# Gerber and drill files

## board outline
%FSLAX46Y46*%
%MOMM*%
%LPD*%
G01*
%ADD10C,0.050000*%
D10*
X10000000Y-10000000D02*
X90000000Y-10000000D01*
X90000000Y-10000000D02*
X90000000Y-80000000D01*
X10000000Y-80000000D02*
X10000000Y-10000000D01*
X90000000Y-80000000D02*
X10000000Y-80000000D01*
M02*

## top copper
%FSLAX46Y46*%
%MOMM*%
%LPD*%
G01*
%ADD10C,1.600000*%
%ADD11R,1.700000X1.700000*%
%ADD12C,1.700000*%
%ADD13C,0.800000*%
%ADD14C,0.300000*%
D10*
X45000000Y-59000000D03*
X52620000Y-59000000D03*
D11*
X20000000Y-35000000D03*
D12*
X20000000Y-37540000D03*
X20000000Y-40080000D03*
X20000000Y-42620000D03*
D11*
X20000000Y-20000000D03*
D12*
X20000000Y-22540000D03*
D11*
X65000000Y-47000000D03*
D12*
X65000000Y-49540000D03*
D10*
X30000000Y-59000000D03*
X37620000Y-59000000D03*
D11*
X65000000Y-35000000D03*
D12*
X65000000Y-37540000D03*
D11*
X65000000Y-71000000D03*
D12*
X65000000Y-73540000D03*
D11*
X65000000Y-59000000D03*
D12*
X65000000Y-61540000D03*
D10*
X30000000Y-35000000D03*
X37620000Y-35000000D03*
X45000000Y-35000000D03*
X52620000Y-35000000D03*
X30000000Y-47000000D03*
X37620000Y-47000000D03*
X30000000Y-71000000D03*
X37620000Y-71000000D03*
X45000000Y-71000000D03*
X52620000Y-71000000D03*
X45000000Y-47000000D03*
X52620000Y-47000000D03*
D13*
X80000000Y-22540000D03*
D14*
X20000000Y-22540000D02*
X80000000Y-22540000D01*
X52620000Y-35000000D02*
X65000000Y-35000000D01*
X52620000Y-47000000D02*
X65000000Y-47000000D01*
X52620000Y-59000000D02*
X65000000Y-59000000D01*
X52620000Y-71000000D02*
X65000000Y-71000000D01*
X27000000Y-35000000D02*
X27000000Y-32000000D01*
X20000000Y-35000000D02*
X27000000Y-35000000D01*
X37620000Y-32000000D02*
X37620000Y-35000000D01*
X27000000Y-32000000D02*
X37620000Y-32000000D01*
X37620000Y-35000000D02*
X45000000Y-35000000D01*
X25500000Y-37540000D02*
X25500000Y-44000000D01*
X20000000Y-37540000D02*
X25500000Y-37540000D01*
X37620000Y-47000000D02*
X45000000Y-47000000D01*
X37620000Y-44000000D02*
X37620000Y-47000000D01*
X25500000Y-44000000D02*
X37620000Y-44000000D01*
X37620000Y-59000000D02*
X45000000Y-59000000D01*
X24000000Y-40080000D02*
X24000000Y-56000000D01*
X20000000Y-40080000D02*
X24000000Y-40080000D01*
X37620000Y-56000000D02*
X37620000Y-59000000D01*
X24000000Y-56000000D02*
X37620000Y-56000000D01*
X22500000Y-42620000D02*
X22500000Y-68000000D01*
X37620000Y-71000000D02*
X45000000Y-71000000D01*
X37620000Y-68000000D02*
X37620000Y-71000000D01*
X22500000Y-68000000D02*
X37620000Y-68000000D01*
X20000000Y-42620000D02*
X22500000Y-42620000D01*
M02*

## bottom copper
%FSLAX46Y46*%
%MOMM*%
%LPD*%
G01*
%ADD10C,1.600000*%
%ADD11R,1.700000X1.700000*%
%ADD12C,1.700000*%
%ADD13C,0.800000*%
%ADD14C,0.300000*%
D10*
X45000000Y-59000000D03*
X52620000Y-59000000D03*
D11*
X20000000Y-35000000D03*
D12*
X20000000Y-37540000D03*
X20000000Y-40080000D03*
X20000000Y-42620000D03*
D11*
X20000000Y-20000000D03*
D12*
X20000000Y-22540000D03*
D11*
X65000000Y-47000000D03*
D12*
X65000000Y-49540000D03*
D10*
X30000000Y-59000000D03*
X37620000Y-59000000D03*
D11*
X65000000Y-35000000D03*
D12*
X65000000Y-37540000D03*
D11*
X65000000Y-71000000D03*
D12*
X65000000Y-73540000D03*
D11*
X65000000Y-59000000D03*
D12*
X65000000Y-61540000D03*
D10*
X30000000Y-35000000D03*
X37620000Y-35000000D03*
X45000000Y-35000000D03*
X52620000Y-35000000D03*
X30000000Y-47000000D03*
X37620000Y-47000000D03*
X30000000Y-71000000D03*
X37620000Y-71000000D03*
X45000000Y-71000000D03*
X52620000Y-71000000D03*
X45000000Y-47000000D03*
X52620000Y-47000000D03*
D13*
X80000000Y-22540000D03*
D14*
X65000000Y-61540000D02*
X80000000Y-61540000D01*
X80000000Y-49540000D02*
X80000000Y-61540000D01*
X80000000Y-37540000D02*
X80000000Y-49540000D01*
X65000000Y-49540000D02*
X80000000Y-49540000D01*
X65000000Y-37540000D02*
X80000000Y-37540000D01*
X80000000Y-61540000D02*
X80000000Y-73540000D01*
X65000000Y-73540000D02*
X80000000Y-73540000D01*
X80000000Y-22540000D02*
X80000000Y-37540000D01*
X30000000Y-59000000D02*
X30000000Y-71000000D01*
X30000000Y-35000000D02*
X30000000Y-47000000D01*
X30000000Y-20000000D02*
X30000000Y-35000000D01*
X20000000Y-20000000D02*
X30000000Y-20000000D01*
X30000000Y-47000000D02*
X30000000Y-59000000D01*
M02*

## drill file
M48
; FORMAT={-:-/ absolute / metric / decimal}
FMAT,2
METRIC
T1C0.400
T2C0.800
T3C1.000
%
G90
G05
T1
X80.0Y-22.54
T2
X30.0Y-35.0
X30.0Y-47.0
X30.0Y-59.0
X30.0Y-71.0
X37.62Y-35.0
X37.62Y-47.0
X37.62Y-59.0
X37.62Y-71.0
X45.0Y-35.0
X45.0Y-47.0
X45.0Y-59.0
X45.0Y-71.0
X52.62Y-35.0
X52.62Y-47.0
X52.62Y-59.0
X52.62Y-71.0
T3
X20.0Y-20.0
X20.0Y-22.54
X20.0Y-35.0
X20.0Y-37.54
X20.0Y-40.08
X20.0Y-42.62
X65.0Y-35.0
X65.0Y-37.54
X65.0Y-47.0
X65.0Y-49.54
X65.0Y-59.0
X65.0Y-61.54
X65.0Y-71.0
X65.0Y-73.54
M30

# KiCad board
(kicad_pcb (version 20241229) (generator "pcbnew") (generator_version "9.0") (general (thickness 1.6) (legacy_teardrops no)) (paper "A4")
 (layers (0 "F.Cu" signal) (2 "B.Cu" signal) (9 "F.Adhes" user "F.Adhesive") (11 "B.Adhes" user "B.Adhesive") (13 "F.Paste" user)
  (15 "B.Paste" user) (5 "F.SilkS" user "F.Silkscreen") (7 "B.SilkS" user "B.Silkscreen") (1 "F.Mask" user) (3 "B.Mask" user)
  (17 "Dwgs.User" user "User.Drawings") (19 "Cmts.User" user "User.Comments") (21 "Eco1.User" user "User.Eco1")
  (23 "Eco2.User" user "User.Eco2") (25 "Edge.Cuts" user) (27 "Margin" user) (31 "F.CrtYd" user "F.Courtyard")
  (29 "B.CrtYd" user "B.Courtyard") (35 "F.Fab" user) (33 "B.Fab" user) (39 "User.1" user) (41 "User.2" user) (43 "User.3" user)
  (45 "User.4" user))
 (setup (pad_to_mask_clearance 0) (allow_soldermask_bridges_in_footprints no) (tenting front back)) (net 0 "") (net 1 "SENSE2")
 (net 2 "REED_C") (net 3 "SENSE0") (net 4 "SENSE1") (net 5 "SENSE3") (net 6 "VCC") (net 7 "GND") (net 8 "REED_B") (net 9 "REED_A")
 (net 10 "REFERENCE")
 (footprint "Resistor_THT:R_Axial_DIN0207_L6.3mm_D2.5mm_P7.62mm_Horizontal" (layer "F.Cu") (at 45 59)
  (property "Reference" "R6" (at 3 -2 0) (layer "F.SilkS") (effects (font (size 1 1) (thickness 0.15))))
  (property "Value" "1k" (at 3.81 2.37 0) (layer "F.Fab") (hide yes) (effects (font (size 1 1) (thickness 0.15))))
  (pad "1" thru_hole circle (at 0 0) (size 1.6 1.6) (drill 0.8) (layers "*.Cu" "*.Mask") (remove_unused_layers no) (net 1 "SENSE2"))
  (pad "2" thru_hole circle (at 7.62 0) (size 1.6 1.6) (drill 0.8) (layers "*.Cu" "*.Mask") (remove_unused_layers no) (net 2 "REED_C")))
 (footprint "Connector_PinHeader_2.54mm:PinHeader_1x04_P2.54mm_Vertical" (layer "F.Cu") (at 20 35)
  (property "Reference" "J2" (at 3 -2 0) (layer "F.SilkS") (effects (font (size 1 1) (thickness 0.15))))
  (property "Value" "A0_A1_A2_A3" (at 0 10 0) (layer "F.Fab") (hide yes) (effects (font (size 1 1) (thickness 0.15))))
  (pad "1" thru_hole rect (at 0 0) (size 1.7 1.7) (drill 1) (layers "*.Cu" "*.Mask") (remove_unused_layers no) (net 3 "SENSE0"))
  (pad "2" thru_hole circle (at 0 2.54) (size 1.7 1.7) (drill 1) (layers "*.Cu" "*.Mask") (remove_unused_layers no) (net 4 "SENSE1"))
  (pad "3" thru_hole circle (at 0 5.08) (size 1.7 1.7) (drill 1) (layers "*.Cu" "*.Mask") (remove_unused_layers no) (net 1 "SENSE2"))
  (pad "4" thru_hole circle (at 0 7.62) (size 1.7 1.7) (drill 1) (layers "*.Cu" "*.Mask") (remove_unused_layers no) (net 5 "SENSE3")))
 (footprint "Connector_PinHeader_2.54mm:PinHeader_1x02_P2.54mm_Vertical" (layer "F.Cu") (at 20 20)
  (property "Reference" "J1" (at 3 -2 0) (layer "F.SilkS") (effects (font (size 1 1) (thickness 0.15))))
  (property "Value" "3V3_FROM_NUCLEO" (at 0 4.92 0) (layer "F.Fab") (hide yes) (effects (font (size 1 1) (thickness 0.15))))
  (pad "1" thru_hole rect (at 0 0) (size 1.7 1.7) (drill 1) (layers "*.Cu" "*.Mask") (remove_unused_layers no) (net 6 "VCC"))
  (pad "2" thru_hole circle (at 0 2.54) (size 1.7 1.7) (drill 1) (layers "*.Cu" "*.Mask") (remove_unused_layers no) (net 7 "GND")))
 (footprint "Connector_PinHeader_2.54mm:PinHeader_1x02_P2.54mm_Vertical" (layer "F.Cu") (at 65 47)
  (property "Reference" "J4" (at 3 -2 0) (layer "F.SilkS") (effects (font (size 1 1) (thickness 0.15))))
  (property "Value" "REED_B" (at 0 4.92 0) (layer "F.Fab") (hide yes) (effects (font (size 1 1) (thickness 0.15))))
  (pad "1" thru_hole rect (at 0 0) (size 1.7 1.7) (drill 1) (layers "*.Cu" "*.Mask") (remove_unused_layers no) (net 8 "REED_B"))
  (pad "2" thru_hole circle (at 0 2.54) (size 1.7 1.7) (drill 1) (layers "*.Cu" "*.Mask") (remove_unused_layers no) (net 7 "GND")))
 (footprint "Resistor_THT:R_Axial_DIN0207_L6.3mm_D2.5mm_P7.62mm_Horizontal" (layer "F.Cu") (at 30 59)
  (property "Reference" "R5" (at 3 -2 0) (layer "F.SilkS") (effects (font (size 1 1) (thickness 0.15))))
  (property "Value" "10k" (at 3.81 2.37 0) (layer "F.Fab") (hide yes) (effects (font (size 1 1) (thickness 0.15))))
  (pad "1" thru_hole circle (at 0 0) (size 1.6 1.6) (drill 0.8) (layers "*.Cu" "*.Mask") (remove_unused_layers no) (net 6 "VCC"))
  (pad "2" thru_hole circle (at 7.62 0) (size 1.6 1.6) (drill 0.8) (layers "*.Cu" "*.Mask") (remove_unused_layers no) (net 1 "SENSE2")))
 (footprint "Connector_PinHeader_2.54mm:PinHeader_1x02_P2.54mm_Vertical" (layer "F.Cu") (at 65 35)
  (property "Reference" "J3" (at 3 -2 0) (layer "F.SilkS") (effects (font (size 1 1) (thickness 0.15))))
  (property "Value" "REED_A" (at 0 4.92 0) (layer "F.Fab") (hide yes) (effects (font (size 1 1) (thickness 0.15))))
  (pad "1" thru_hole rect (at 0 0) (size 1.7 1.7) (drill 1) (layers "*.Cu" "*.Mask") (remove_unused_layers no) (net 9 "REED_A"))
  (pad "2" thru_hole circle (at 0 2.54) (size 1.7 1.7) (drill 1) (layers "*.Cu" "*.Mask") (remove_unused_layers no) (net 7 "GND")))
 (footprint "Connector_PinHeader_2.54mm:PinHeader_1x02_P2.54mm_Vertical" (layer "F.Cu") (at 65 71)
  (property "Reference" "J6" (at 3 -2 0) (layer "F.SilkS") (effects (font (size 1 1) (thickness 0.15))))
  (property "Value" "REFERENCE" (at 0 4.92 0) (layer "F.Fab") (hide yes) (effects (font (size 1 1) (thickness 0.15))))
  (pad "1" thru_hole rect (at 0 0) (size 1.7 1.7) (drill 1) (layers "*.Cu" "*.Mask") (remove_unused_layers no) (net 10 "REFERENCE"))
  (pad "2" thru_hole circle (at 0 2.54) (size 1.7 1.7) (drill 1) (layers "*.Cu" "*.Mask") (remove_unused_layers no) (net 7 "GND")))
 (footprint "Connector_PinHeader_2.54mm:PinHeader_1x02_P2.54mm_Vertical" (layer "F.Cu") (at 65 59)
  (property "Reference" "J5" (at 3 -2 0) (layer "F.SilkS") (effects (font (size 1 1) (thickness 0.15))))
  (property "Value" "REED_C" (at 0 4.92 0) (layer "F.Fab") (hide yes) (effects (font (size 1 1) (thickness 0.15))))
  (pad "1" thru_hole rect (at 0 0) (size 1.7 1.7) (drill 1) (layers "*.Cu" "*.Mask") (remove_unused_layers no) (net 2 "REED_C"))
  (pad "2" thru_hole circle (at 0 2.54) (size 1.7 1.7) (drill 1) (layers "*.Cu" "*.Mask") (remove_unused_layers no) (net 7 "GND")))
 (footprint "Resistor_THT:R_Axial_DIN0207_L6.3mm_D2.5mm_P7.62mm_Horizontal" (layer "F.Cu") (at 30 35)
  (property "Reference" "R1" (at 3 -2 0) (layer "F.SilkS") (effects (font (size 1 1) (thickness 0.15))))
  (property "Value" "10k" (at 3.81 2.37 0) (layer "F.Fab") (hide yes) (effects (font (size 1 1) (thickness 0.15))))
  (pad "1" thru_hole circle (at 0 0) (size 1.6 1.6) (drill 0.8) (layers "*.Cu" "*.Mask") (remove_unused_layers no) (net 6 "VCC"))
  (pad "2" thru_hole circle (at 7.62 0) (size 1.6 1.6) (drill 0.8) (layers "*.Cu" "*.Mask") (remove_unused_layers no) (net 3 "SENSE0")))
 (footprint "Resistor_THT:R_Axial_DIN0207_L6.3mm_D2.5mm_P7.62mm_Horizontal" (layer "F.Cu") (at 45 35)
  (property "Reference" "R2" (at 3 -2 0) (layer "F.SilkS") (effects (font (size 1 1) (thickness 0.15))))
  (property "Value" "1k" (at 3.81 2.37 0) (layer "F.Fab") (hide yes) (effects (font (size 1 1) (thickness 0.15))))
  (pad "1" thru_hole circle (at 0 0) (size 1.6 1.6) (drill 0.8) (layers "*.Cu" "*.Mask") (remove_unused_layers no) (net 3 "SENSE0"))
  (pad "2" thru_hole circle (at 7.62 0) (size 1.6 1.6) (drill 0.8) (layers "*.Cu" "*.Mask") (remove_unused_layers no) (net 9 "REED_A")))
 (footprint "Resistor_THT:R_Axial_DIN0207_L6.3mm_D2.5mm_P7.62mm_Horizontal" (layer "F.Cu") (at 30 47)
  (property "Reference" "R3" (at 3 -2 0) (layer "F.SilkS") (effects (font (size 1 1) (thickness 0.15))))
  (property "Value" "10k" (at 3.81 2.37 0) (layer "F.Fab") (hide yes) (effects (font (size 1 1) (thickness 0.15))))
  (pad "1" thru_hole circle (at 0 0) (size 1.6 1.6) (drill 0.8) (layers "*.Cu" "*.Mask") (remove_unused_layers no) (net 6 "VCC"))
  (pad "2" thru_hole circle (at 7.62 0) (size 1.6 1.6) (drill 0.8) (layers "*.Cu" "*.Mask") (remove_unused_layers no) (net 4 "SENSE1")))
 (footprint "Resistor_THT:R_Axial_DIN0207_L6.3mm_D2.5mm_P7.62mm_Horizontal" (layer "F.Cu") (at 30 71)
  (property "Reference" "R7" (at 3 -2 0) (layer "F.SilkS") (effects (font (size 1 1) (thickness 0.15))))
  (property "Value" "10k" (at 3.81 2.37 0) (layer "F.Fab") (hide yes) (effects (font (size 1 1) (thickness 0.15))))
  (pad "1" thru_hole circle (at 0 0) (size 1.6 1.6) (drill 0.8) (layers "*.Cu" "*.Mask") (remove_unused_layers no) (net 6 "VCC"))
  (pad "2" thru_hole circle (at 7.62 0) (size 1.6 1.6) (drill 0.8) (layers "*.Cu" "*.Mask") (remove_unused_layers no) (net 5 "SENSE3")))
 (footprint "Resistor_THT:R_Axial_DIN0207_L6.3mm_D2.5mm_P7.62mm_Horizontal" (layer "F.Cu") (at 45 71)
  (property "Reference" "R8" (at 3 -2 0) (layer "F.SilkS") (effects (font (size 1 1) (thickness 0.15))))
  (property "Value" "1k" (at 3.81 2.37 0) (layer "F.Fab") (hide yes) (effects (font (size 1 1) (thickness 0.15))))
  (pad "1" thru_hole circle (at 0 0) (size 1.6 1.6) (drill 0.8) (layers "*.Cu" "*.Mask") (remove_unused_layers no) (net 5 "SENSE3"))
  (pad "2" thru_hole circle (at 7.62 0) (size 1.6 1.6) (drill 0.8) (layers "*.Cu" "*.Mask") (remove_unused_layers no) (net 10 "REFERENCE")))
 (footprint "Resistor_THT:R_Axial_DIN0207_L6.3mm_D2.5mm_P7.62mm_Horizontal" (layer "F.Cu") (at 45 47)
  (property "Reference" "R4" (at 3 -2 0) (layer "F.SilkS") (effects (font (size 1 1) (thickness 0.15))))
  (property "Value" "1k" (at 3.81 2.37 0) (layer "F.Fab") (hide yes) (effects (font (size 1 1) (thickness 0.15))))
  (pad "1" thru_hole circle (at 0 0) (size 1.6 1.6) (drill 0.8) (layers "*.Cu" "*.Mask") (remove_unused_layers no) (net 4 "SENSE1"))
  (pad "2" thru_hole circle (at 7.62 0) (size 1.6 1.6) (drill 0.8) (layers "*.Cu" "*.Mask") (remove_unused_layers no) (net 8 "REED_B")))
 (gr_line (start 10 10) (end 90 10) (stroke (width 0.05) (type default)) (layer "Edge.Cuts"))
 (gr_line (start 90 10) (end 90 80) (stroke (width 0.05) (type default)) (layer "Edge.Cuts"))
 (gr_line (start 10 80) (end 10 10) (stroke (width 0.05) (type default)) (layer "Edge.Cuts"))
 (gr_line (start 90 80) (end 10 80) (stroke (width 0.05) (type default)) (layer "Edge.Cuts"))
 (segment (start 20 22.54) (end 80 22.54) (width 0.3) (layer "F.Cu") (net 7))
 (via (at 80 22.54) (size 0.8) (drill 0.4) (layers "F.Cu" "B.Cu") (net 7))
 (segment (start 65 61.54) (end 80 61.54) (width 0.3) (layer "B.Cu") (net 7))
 (segment (start 80 49.54) (end 80 61.54) (width 0.3) (layer "B.Cu") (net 7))
 (segment (start 80 37.54) (end 80 49.54) (width 0.3) (layer "B.Cu") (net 7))
 (segment (start 65 49.54) (end 80 49.54) (width 0.3) (layer "B.Cu") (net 7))
 (segment (start 65 37.54) (end 80 37.54) (width 0.3) (layer "B.Cu") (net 7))
 (segment (start 80 61.54) (end 80 73.54) (width 0.3) (layer "B.Cu") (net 7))
 (segment (start 65 73.54) (end 80 73.54) (width 0.3) (layer "B.Cu") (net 7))
 (segment (start 80 22.54) (end 80 37.54) (width 0.3) (layer "B.Cu") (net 7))
 (segment (start 52.62 35) (end 65 35) (width 0.3) (layer "F.Cu") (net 9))
 (segment (start 52.62 47) (end 65 47) (width 0.3) (layer "F.Cu") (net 8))
 (segment (start 52.62 59) (end 65 59) (width 0.3) (layer "F.Cu") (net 2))
 (segment (start 52.62 71) (end 65 71) (width 0.3) (layer "F.Cu") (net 10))
 (segment (start 27 35) (end 27 32) (width 0.3) (layer "F.Cu") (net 3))
 (segment (start 20 35) (end 27 35) (width 0.3) (layer "F.Cu") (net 3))
 (segment (start 37.62 32) (end 37.62 35) (width 0.3) (layer "F.Cu") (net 3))
 (segment (start 27 32) (end 37.62 32) (width 0.3) (layer "F.Cu") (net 3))
 (segment (start 37.62 35) (end 45 35) (width 0.3) (layer "F.Cu") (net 3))
 (segment (start 25.5 37.54) (end 25.5 44) (width 0.3) (layer "F.Cu") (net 4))
 (segment (start 20 37.54) (end 25.5 37.54) (width 0.3) (layer "F.Cu") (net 4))
 (segment (start 37.62 47) (end 45 47) (width 0.3) (layer "F.Cu") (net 4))
 (segment (start 37.62 44) (end 37.62 47) (width 0.3) (layer "F.Cu") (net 4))
 (segment (start 25.5 44) (end 37.62 44) (width 0.3) (layer "F.Cu") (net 4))
 (segment (start 37.62 59) (end 45 59) (width 0.3) (layer "F.Cu") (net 1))
 (segment (start 24 40.08) (end 24 56) (width 0.3) (layer "F.Cu") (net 1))
 (segment (start 20 40.08) (end 24 40.08) (width 0.3) (layer "F.Cu") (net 1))
 (segment (start 37.62 56) (end 37.62 59) (width 0.3) (layer "F.Cu") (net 1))
 (segment (start 24 56) (end 37.62 56) (width 0.3) (layer "F.Cu") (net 1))
 (segment (start 22.5 42.62) (end 22.5 68) (width 0.3) (layer "F.Cu") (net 5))
 (segment (start 37.62 71) (end 45 71) (width 0.3) (layer "F.Cu") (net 5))
 (segment (start 37.62 68) (end 37.62 71) (width 0.3) (layer "F.Cu") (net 5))
 (segment (start 22.5 68) (end 37.62 68) (width 0.3) (layer "F.Cu") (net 5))
 (segment (start 20 42.62) (end 22.5 42.62) (width 0.3) (layer "F.Cu") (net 5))
 (segment (start 30 59) (end 30 71) (width 0.3) (layer "B.Cu") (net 6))
 (segment (start 30 35) (end 30 47) (width 0.3) (layer "B.Cu") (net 6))
 (segment (start 30 20) (end 30 35) (width 0.3) (layer "B.Cu") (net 6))
 (segment (start 20 20) (end 30 20) (width 0.3) (layer "B.Cu") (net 6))
 (segment (start 30 47) (end 30 59) (width 0.3) (layer "B.Cu") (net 6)))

